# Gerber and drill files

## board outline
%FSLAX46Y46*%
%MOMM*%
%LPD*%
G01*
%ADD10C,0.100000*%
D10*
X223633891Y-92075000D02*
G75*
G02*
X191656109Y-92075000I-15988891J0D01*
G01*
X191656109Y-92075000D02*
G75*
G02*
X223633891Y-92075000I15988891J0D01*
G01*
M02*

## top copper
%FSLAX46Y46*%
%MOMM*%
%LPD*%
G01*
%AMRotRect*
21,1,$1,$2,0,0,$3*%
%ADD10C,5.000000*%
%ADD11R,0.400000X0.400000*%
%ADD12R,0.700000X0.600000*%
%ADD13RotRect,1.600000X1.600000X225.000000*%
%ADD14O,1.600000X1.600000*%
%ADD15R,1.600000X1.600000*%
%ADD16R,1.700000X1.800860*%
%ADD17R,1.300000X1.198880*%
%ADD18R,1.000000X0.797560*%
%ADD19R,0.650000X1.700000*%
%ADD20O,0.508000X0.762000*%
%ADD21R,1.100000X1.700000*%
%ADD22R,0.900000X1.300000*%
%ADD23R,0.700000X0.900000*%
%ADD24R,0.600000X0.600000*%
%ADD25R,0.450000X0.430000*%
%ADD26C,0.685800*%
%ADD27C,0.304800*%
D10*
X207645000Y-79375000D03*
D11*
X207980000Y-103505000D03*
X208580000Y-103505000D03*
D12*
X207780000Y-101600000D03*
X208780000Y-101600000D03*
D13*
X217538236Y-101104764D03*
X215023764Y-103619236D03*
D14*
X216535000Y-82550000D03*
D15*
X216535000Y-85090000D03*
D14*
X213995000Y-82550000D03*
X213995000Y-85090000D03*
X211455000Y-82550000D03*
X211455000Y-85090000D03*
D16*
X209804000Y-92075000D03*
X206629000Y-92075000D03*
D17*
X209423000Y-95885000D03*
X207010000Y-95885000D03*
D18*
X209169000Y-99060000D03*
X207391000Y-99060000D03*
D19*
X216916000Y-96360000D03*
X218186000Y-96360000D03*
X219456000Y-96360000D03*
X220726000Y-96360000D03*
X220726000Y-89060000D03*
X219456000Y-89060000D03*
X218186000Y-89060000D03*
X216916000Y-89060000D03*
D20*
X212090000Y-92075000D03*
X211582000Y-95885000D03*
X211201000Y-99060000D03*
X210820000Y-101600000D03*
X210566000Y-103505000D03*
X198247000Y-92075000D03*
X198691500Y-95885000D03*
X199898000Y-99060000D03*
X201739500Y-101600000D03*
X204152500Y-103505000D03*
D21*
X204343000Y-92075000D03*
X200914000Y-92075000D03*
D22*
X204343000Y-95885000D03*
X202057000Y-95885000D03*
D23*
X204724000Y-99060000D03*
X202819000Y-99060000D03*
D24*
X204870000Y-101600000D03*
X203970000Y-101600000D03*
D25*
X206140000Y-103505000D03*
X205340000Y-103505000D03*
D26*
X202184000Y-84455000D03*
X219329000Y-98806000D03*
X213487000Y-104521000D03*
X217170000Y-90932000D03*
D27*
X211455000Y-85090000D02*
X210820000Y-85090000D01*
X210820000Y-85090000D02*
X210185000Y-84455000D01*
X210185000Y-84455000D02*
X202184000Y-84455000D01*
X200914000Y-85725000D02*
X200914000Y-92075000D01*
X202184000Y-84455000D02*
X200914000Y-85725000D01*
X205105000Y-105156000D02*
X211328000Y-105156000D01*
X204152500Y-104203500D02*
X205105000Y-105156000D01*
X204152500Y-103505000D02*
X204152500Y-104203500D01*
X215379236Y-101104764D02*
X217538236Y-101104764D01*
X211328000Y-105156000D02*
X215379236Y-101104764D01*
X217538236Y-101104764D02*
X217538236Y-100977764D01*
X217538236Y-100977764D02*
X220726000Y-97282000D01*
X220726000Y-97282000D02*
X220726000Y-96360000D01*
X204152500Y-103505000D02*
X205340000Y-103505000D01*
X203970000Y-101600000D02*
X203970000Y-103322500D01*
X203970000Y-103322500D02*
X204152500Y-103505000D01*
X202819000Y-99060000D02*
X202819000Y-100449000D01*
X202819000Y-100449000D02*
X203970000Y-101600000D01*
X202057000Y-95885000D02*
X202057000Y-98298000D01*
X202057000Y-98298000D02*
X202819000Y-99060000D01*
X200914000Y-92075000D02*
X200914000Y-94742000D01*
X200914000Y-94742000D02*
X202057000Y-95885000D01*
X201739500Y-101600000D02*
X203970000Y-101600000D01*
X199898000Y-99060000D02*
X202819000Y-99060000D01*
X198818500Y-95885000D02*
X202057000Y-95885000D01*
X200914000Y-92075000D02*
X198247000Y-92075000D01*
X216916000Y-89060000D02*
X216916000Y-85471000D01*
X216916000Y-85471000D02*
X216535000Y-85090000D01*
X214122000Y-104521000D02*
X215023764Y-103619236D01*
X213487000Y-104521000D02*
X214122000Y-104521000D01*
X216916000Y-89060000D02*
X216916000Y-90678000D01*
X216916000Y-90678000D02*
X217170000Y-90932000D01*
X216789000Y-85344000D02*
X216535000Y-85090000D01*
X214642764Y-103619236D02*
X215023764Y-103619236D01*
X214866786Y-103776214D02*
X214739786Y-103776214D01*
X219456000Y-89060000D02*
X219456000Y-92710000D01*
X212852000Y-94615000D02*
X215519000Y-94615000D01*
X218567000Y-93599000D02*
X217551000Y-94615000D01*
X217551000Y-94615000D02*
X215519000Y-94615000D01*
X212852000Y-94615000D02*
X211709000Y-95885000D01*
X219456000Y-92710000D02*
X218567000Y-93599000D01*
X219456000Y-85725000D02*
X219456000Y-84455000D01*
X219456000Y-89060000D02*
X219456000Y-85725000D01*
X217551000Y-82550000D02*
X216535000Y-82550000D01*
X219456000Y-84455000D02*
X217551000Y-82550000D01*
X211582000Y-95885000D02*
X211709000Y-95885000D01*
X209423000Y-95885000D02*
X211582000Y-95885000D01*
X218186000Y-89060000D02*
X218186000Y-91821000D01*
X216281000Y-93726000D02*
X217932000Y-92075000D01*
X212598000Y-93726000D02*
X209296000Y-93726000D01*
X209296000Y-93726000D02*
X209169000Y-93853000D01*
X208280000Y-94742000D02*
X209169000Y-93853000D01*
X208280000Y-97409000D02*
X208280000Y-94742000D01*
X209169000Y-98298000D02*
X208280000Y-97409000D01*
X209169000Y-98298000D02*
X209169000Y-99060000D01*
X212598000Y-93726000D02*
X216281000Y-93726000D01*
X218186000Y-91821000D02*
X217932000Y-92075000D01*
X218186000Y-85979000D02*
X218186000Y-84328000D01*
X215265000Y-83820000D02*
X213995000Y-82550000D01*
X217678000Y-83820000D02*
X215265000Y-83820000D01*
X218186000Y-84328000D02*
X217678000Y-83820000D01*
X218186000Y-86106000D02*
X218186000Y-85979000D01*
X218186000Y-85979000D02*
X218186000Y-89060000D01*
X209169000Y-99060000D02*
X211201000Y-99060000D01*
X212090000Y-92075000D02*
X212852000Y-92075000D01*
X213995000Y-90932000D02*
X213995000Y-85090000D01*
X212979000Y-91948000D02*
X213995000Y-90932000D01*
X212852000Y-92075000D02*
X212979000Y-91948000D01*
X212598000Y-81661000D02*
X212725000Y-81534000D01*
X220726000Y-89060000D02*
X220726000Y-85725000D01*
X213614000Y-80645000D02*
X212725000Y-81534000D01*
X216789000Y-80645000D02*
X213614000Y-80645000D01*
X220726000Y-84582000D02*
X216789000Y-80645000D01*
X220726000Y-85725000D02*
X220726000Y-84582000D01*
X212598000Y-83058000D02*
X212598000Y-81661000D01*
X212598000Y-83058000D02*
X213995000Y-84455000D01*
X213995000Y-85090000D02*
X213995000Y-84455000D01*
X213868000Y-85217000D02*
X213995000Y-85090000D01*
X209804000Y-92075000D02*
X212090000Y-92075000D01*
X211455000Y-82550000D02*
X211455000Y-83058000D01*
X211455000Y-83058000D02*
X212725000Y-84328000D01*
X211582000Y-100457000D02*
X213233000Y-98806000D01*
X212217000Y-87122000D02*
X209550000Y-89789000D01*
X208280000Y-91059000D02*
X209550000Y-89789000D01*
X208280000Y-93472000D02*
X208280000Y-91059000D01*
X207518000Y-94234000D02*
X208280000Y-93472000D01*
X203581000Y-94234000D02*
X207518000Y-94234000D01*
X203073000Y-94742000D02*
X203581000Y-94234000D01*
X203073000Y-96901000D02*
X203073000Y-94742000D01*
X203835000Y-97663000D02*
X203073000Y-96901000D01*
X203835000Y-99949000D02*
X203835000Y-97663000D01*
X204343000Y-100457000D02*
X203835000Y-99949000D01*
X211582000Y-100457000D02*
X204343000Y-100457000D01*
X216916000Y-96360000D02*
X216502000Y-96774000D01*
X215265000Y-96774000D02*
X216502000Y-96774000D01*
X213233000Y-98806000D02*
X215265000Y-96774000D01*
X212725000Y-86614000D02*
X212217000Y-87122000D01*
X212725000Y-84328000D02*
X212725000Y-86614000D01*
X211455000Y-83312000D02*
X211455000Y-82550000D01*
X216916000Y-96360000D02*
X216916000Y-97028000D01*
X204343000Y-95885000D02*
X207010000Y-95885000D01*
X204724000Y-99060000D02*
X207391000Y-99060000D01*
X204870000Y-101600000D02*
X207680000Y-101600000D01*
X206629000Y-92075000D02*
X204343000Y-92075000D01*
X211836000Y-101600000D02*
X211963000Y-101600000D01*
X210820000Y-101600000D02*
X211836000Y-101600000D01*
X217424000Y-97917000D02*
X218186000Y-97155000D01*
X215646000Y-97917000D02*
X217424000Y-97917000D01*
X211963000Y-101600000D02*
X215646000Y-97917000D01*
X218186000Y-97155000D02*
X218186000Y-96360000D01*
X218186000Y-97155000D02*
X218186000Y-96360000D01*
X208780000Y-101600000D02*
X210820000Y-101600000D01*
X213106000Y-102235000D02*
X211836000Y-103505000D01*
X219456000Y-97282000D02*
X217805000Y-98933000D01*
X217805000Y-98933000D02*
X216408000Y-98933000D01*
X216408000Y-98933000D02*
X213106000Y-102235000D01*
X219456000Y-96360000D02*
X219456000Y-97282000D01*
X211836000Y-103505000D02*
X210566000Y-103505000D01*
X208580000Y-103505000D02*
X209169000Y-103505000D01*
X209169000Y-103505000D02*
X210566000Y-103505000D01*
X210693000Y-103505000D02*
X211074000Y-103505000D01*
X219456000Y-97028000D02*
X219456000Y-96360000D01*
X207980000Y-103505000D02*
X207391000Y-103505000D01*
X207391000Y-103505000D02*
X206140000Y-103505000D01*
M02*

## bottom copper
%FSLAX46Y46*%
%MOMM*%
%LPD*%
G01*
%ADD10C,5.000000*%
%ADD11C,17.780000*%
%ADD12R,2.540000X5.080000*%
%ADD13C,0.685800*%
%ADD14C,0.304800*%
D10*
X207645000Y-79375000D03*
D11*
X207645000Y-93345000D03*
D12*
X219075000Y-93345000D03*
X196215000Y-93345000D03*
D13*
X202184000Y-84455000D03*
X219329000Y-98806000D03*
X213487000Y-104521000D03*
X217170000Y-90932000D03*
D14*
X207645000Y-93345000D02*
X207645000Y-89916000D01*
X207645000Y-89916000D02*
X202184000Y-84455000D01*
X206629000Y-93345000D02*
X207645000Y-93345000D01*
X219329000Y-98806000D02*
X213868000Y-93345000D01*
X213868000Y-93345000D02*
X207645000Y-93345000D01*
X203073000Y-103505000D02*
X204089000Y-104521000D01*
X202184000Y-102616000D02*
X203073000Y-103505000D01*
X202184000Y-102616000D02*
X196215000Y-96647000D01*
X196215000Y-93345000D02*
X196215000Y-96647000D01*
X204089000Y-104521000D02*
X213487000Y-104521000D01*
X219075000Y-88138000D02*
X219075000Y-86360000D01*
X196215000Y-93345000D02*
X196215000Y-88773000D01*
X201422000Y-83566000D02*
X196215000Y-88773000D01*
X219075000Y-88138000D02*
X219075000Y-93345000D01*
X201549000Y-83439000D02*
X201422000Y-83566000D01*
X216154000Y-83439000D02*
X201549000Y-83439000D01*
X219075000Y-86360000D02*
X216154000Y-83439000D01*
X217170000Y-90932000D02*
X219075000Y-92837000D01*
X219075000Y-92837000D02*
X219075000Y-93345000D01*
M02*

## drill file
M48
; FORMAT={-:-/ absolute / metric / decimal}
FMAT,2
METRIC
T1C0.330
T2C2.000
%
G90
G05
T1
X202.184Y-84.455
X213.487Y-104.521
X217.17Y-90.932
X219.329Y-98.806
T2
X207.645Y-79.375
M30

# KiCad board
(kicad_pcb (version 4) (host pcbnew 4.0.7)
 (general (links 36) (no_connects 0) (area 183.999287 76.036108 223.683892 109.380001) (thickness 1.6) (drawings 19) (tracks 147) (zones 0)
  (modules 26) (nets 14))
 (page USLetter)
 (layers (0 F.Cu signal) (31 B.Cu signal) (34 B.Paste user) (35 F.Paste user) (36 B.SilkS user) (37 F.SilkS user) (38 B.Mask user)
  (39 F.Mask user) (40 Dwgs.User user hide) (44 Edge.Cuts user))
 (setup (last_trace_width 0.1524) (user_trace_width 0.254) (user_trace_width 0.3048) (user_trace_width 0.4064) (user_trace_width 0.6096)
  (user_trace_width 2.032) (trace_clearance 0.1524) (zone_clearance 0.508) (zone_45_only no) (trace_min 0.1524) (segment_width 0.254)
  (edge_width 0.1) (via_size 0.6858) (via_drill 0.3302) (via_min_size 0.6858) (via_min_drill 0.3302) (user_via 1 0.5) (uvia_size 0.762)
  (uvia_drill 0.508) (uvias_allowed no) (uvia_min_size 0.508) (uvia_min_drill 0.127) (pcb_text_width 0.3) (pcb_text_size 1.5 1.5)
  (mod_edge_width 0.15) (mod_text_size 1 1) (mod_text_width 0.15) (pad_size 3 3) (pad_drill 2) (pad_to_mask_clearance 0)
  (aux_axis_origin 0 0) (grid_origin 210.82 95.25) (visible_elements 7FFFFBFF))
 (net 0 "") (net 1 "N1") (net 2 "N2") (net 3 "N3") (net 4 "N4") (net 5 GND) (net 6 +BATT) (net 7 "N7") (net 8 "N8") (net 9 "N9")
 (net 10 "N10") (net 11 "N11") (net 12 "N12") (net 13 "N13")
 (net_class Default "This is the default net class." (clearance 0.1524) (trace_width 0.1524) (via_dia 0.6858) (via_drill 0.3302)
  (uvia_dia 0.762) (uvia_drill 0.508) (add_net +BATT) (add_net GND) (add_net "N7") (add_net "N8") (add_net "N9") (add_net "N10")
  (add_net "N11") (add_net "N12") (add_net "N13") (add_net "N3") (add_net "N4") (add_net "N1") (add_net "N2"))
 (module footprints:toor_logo (layer F.Cu) (at 205.232 88.392)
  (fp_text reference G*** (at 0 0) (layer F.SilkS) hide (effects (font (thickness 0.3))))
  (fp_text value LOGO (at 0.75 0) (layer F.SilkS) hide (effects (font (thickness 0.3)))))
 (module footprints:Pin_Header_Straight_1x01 (layer F.Cu) (at 207.645 79.375)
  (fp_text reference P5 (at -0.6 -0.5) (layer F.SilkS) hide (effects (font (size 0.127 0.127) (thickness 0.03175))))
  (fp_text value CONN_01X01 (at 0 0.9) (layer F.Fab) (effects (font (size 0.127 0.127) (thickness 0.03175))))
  (pad 1 thru_hole circle (at 0 0) (size 5 5) (drill 2) (layers *.Cu *.Mask)))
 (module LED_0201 (layer F.Cu) (at 208.28 103.505)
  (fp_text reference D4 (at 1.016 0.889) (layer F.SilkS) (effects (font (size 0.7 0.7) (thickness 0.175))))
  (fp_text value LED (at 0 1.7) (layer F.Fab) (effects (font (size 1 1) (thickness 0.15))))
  (pad 1 smd rect (at -0.3 0) (size 0.4 0.4) (layers F.Cu F.Paste F.Mask) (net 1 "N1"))
  (pad 2 smd rect (at 0.3 0) (size 0.4 0.4) (layers F.Cu F.Paste F.Mask) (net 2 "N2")))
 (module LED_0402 (layer F.Cu) (at 208.28 101.6)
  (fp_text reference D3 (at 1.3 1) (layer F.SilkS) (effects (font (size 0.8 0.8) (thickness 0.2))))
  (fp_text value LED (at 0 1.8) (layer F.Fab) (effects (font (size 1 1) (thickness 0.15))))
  (pad 1 smd rect (at -0.5 0) (size 0.7 0.6) (layers F.Cu F.Paste F.Mask) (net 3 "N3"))
  (pad 2 smd rect (at 0.5 0) (size 0.7 0.6) (layers F.Cu F.Paste F.Mask) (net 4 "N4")))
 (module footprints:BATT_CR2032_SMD (layer B.Cu) (at 207.645 93.345 180)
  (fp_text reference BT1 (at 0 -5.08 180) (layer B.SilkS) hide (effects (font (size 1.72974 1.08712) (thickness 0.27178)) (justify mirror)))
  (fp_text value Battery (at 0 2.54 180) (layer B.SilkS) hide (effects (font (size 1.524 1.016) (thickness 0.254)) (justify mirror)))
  (pad 2 smd circle (at 0 0 180) (size 17.78 17.78) (layers B.Cu B.Paste B.Mask) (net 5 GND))
  (pad 1 smd rect (at -11.43 0 180) (size 2.54 5.08) (layers B.Cu B.Paste B.Mask) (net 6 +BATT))
  (pad 1 smd rect (at 11.43 0 180) (size 2.54 5.08) (layers B.Cu B.Paste B.Mask) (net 6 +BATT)))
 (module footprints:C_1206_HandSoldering (layer F.Cu) (at 216.281 102.362 225)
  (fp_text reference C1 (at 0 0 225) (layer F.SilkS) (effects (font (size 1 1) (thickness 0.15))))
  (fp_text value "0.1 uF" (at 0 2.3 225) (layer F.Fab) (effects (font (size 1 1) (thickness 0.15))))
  (pad 1 smd rect (at -1.778 0 225) (size 1.6 1.6) (layers F.Cu F.Paste F.Mask) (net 5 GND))
  (pad 2 smd rect (at 1.778 0 225) (size 1.6 1.6) (layers F.Cu F.Paste F.Mask) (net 6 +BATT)))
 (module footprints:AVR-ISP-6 (layer F.Cu) (at 216.535 82.55 270)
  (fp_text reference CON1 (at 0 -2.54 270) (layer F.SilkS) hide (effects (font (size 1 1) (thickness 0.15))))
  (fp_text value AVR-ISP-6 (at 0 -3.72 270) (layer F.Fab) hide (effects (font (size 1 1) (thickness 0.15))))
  (pad 1 smd oval (at 0 0 270) (size 1.6 1.6) (layers F.Cu F.Paste F.Mask) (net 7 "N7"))
  (pad 2 smd rect (at 2.54 0 270) (size 1.6 1.6) (layers F.Cu F.Paste F.Mask) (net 6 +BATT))
  (pad 3 smd oval (at 0 2.54 270) (size 1.6 1.6) (layers F.Cu F.Paste F.Mask) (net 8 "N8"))
  (pad 4 smd oval (at 2.54 2.54 270) (size 1.6 1.6) (layers F.Cu F.Paste F.Mask) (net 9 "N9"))
  (pad 5 smd oval (at 0 5.08 270) (size 1.6 1.6) (layers F.Cu F.Paste F.Mask) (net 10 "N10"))
  (pad 6 smd oval (at 2.54 5.08 270) (size 1.6 1.6) (layers F.Cu F.Paste F.Mask) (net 5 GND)))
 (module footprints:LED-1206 (layer F.Cu) (at 208.28 92.075)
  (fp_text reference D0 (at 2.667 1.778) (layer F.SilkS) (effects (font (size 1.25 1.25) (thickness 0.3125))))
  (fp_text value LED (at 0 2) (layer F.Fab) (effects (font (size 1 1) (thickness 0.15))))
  (pad 2 smd rect (at 1.524 0 180) (size 1.7 1.80086) (layers F.Cu F.Paste F.Mask) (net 9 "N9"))
  (pad 1 smd rect (at -1.651 0 180) (size 1.7 1.80086) (layers F.Cu F.Paste F.Mask) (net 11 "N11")))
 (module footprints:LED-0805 (layer F.Cu) (at 208.28 95.885)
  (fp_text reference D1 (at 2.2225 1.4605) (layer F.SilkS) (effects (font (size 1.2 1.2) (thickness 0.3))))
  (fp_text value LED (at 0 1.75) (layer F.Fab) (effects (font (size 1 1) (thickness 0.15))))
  (pad 2 smd rect (at 1.143 0 180) (size 1.3 1.19888) (layers F.Cu F.Paste F.Mask) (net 7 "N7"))
  (pad 1 smd rect (at -1.27 0 180) (size 1.3 1.19888) (layers F.Cu F.Paste F.Mask) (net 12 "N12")))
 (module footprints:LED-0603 (layer F.Cu) (at 208.28 99.06)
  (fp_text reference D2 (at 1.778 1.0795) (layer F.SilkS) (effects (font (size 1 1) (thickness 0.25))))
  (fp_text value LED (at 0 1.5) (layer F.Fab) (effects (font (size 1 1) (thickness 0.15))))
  (pad 2 smd rect (at 0.889 0 180) (size 1 0.79756) (layers F.Cu F.Paste F.Mask) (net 8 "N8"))
  (pad 1 smd rect (at -0.889 0 180) (size 1 0.79756) (layers F.Cu F.Paste F.Mask) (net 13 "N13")))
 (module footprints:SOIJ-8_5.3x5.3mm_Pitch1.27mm (layer F.Cu) (at 218.821 92.71 90)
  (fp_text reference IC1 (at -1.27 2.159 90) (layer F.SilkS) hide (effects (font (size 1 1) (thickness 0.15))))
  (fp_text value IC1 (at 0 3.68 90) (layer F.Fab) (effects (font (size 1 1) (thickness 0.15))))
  (pad 1 smd rect (at -3.65 -1.905 90) (size 1.7 0.65) (layers F.Cu F.Paste F.Mask) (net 10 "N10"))
  (pad 2 smd rect (at -3.65 -0.635 90) (size 1.7 0.65) (layers F.Cu F.Paste F.Mask) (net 4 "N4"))
  (pad 3 smd rect (at -3.65 0.635 90) (size 1.7 0.65) (layers F.Cu F.Paste F.Mask) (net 2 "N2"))
  (pad 4 smd rect (at -3.65 1.905 90) (size 1.7 0.65) (layers F.Cu F.Paste F.Mask) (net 5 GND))
  (pad 5 smd rect (at 3.65 1.905 90) (size 1.7 0.65) (layers F.Cu F.Paste F.Mask) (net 9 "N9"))
  (pad 6 smd rect (at 3.65 0.635 90) (size 1.7 0.65) (layers F.Cu F.Paste F.Mask) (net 7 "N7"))
  (pad 7 smd rect (at 3.65 -0.635 90) (size 1.7 0.65) (layers F.Cu F.Paste F.Mask) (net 8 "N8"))
  (pad 8 smd rect (at 3.65 -1.905 90) (size 1.7 0.65) (layers F.Cu F.Paste F.Mask) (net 6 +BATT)))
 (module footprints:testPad (layer F.Cu) (at 212.09 92.075)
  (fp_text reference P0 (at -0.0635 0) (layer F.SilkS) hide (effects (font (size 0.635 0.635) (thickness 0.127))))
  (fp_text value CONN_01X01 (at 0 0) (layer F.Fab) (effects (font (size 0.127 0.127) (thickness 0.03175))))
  (pad 1 smd oval (at 0 0) (size 0.508 0.762) (layers F.Cu F.Paste F.Mask) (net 9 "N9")))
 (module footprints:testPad (layer F.Cu) (at 211.582 95.885)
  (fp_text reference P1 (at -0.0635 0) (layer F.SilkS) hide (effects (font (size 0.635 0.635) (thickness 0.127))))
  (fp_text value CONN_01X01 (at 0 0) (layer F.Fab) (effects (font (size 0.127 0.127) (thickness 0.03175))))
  (pad 1 smd oval (at 0 0) (size 0.508 0.762) (layers F.Cu F.Paste F.Mask) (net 7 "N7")))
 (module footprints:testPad (layer F.Cu) (at 211.201 99.06)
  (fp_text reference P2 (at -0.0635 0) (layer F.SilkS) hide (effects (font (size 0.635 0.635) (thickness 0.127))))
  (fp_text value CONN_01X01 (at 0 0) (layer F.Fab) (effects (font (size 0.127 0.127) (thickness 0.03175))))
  (pad 1 smd oval (at 0 0) (size 0.508 0.762) (layers F.Cu F.Paste F.Mask) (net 8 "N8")))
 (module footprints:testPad (layer F.Cu) (at 210.82 101.6)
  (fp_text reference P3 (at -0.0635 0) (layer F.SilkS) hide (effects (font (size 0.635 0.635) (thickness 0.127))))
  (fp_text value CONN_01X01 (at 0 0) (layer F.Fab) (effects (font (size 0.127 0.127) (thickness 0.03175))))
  (pad 1 smd oval (at 0 0) (size 0.508 0.762) (layers F.Cu F.Paste F.Mask) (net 4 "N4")))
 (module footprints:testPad (layer F.Cu) (at 210.566 103.505)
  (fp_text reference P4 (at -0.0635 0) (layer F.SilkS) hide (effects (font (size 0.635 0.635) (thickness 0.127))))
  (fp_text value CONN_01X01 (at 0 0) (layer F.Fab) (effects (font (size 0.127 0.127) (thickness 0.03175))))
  (pad 1 smd oval (at 0 0) (size 0.508 0.762) (layers F.Cu F.Paste F.Mask) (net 2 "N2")))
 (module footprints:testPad (layer F.Cu) (at 198.247 92.075)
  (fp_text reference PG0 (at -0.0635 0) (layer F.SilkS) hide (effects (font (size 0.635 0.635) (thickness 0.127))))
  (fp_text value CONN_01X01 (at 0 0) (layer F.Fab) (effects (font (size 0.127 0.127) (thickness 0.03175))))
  (pad 1 smd oval (at 0 0) (size 0.508 0.762) (layers F.Cu F.Paste F.Mask) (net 5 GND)))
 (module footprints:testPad (layer F.Cu) (at 198.6915 95.885)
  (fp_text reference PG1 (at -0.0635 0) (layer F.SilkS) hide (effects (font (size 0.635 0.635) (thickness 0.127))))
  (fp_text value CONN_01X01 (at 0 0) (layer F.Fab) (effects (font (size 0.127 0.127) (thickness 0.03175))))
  (pad 1 smd oval (at 0 0) (size 0.508 0.762) (layers F.Cu F.Paste F.Mask) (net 5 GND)))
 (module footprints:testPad (layer F.Cu) (at 199.898 99.06)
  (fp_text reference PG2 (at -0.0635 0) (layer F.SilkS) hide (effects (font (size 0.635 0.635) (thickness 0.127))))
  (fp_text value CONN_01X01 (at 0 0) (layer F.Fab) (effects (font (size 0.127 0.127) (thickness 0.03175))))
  (pad 1 smd oval (at 0 0) (size 0.508 0.762) (layers F.Cu F.Paste F.Mask) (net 5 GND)))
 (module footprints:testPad (layer F.Cu) (at 201.7395 101.6)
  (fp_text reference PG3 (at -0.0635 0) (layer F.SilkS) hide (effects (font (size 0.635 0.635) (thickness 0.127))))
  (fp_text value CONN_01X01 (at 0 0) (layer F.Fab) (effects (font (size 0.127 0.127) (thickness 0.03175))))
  (pad 1 smd oval (at 0 0) (size 0.508 0.762) (layers F.Cu F.Paste F.Mask) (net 5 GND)))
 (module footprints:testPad (layer F.Cu) (at 204.1525 103.505)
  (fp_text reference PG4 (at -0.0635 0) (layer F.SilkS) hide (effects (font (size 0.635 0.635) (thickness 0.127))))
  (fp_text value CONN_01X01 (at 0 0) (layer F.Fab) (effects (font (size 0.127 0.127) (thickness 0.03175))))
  (pad 1 smd oval (at 0 0) (size 0.508 0.762) (layers F.Cu F.Paste F.Mask) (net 5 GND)))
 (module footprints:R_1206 (layer F.Cu) (at 202.565 92.075 180)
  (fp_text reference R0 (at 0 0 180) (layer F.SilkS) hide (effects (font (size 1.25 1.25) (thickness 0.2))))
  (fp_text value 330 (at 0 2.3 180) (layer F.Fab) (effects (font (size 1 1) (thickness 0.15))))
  (pad 1 smd rect (at -1.778 0 180) (size 1.1 1.7) (layers F.Cu F.Paste F.Mask) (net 11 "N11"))
  (pad 2 smd rect (at 1.651 0 180) (size 1.1 1.7) (layers F.Cu F.Paste F.Mask) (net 5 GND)))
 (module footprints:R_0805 (layer F.Cu) (at 203.2 95.885 180)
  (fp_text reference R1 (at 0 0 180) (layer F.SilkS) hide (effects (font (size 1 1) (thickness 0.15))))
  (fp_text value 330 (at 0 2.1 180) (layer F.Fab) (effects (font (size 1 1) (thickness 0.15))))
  (pad 1 smd rect (at -1.143 0 180) (size 0.9 1.3) (layers F.Cu F.Paste F.Mask) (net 12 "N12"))
  (pad 2 smd rect (at 1.143 0 180) (size 0.9 1.3) (layers F.Cu F.Paste F.Mask) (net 5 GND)))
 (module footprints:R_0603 (layer F.Cu) (at 203.835 99.06 180)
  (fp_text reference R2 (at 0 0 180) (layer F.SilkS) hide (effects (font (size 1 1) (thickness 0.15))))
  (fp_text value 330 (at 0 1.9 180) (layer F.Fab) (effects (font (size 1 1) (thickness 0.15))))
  (pad 1 smd rect (at -0.889 0 180) (size 0.7 0.9) (layers F.Cu F.Paste F.Mask) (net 13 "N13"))
  (pad 2 smd rect (at 1.016 0 180) (size 0.7 0.9) (layers F.Cu F.Paste F.Mask) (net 5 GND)))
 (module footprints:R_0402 (layer F.Cu) (at 204.47 101.6 180)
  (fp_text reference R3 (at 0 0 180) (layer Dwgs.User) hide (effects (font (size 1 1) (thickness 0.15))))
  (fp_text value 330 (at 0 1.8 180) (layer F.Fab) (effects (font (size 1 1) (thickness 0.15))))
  (pad 1 smd rect (at -0.4 0 180) (size 0.6 0.6) (layers F.Cu F.Paste F.Mask) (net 3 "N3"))
  (pad 2 smd rect (at 0.5 0 180) (size 0.6 0.6) (layers F.Cu F.Paste F.Mask) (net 5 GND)))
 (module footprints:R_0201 (layer F.Cu) (at 205.74 103.505 180)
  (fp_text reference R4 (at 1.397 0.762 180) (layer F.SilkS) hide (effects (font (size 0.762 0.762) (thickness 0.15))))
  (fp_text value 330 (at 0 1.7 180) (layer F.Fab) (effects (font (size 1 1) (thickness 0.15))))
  (pad 1 smd rect (at -0.4 0 180) (size 0.45 0.43) (layers F.Cu F.Paste F.Mask) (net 1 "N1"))
  (pad 2 smd rect (at 0.4 0 180) (size 0.45 0.43) (layers F.Cu F.Paste F.Mask) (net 5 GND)))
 (gr_circle (center 207.645 92.075) (end 191.77 90.17) (layer Edge.Cuts) (width 0.1))
 (segment (start 211.455 85.09) (end 210.82 85.09) (width 0.3048) (layer F.Cu) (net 5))
 (segment (start 210.82 85.09) (end 210.185 84.455) (width 0.3048) (layer F.Cu) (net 5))
 (segment (start 210.185 84.455) (end 202.184 84.455) (width 0.3048) (layer F.Cu) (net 5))
 (segment (start 207.645 93.345) (end 207.645 89.916) (width 0.3048) (layer B.Cu) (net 5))
 (segment (start 207.645 89.916) (end 202.184 84.455) (width 0.3048) (layer B.Cu) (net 5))
 (segment (start 200.914 85.725) (end 200.914 92.075) (width 0.3048) (layer F.Cu) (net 5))
 (segment (start 202.184 84.455) (end 200.914 85.725) (width 0.3048) (layer F.Cu) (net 5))
 (via (at 202.184 84.455) (size 0.6858) (drill 0.3302) (layers F.Cu B.Cu) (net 5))
 (segment (start 205.105 105.156) (end 211.328 105.156) (width 0.3048) (layer F.Cu) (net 5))
 (segment (start 204.1525 104.2035) (end 205.105 105.156) (width 0.3048) (layer F.Cu) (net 5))
 (segment (start 204.1525 103.505) (end 204.1525 104.2035) (width 0.3048) (layer F.Cu) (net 5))
 (segment (start 215.379236 101.104764) (end 217.538236 101.104764) (width 0.3048) (layer F.Cu) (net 5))
 (segment (start 211.328 105.156) (end 215.379236 101.104764) (width 0.3048) (layer F.Cu) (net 5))
 (segment (start 217.538236 101.104764) (end 217.538236 100.977764) (width 0.3048) (layer F.Cu) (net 5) (status 30))
 (segment (start 217.538236 100.977764) (end 220.726 97.282) (width 0.3048) (layer F.Cu) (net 5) (status 10))
 (segment (start 220.726 97.282) (end 220.726 96.36) (width 0.3048) (layer F.Cu) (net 5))
 (segment (start 204.1525 103.505) (end 205.34 103.505) (width 0.3048) (layer F.Cu) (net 5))
 (segment (start 203.97 101.6) (end 203.97 103.3225) (width 0.3048) (layer F.Cu) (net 5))
 (segment (start 203.97 103.3225) (end 204.1525 103.505) (width 0.3048) (layer F.Cu) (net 5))
 (segment (start 206.629 93.345) (end 207.645 93.345) (width 0.3048) (layer B.Cu) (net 5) (status 30))
 (segment (start 219.329 98.806) (end 213.868 93.345) (width 0.3048) (layer B.Cu) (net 5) (status 20))
 (via (at 219.329 98.806) (size 0.6858) (drill 0.3302) (layers F.Cu B.Cu) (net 5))
 (segment (start 213.868 93.345) (end 207.645 93.345) (width 0.3048) (layer B.Cu) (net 5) (status 30))
 (segment (start 202.819 99.06) (end 202.819 100.449) (width 0.3048) (layer F.Cu) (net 5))
 (segment (start 202.819 100.449) (end 203.97 101.6) (width 0.3048) (layer F.Cu) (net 5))
 (segment (start 202.057 95.885) (end 202.057 98.298) (width 0.3048) (layer F.Cu) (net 5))
 (segment (start 202.057 98.298) (end 202.819 99.06) (width 0.3048) (layer F.Cu) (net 5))
 (segment (start 200.914 92.075) (end 200.914 94.742) (width 0.3048) (layer F.Cu) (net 5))
 (segment (start 200.914 94.742) (end 202.057 95.885) (width 0.3048) (layer F.Cu) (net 5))
 (segment (start 201.7395 101.6) (end 203.97 101.6) (width 0.3048) (layer F.Cu) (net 5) (status 10))
 (segment (start 199.898 99.06) (end 202.819 99.06) (width 0.3048) (layer F.Cu) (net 5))
 (segment (start 198.8185 95.885) (end 202.057 95.885) (width 0.3048) (layer F.Cu) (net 5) (status 10))
 (segment (start 200.914 92.075) (end 198.247 92.075) (width 0.3048) (layer F.Cu) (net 5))
 (segment (start 216.916 89.06) (end 216.916 85.471) (width 0.3048) (layer F.Cu) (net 6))
 (segment (start 216.916 85.471) (end 216.535 85.09) (width 0.3048) (layer F.Cu) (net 6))
 (segment (start 203.073 103.505) (end 204.089 104.521) (width 0.3048) (layer B.Cu) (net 6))
 (segment (start 202.184 102.616) (end 203.073 103.505) (width 0.3048) (layer B.Cu) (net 6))
 (segment (start 202.184 102.616) (end 196.215 96.647) (width 0.3048) (layer B.Cu) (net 6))
 (segment (start 196.215 93.345) (end 196.215 96.647) (width 0.3048) (layer B.Cu) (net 6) (status 10))
 (segment (start 214.122 104.521) (end 215.023764 103.619236) (width 0.3048) (layer F.Cu) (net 6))
 (segment (start 213.487 104.521) (end 214.122 104.521) (width 0.3048) (layer F.Cu) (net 6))
 (via (at 213.487 104.521) (size 0.6858) (drill 0.3302) (layers F.Cu B.Cu) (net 6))
 (segment (start 204.089 104.521) (end 213.487 104.521) (width 0.3048) (layer B.Cu) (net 6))
 (segment (start 219.075 88.138) (end 219.075 86.36) (width 0.3048) (layer B.Cu) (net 6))
 (segment (start 196.215 93.345) (end 196.215 88.773) (width 0.3048) (layer B.Cu) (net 6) (status 20))
 (segment (start 201.422 83.566) (end 196.215 88.773) (width 0.3048) (layer B.Cu) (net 6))
 (segment (start 219.075 88.138) (end 219.075 93.345) (width 0.3048) (layer B.Cu) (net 6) (status 10))
 (segment (start 201.549 83.439) (end 201.422 83.566) (width 0.3048) (layer B.Cu) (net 6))
 (segment (start 216.154 83.439) (end 201.549 83.439) (width 0.3048) (layer B.Cu) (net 6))
 (segment (start 219.075 86.36) (end 216.154 83.439) (width 0.3048) (layer B.Cu) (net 6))
 (segment (start 216.916 89.06) (end 216.916 90.678) (width 0.3048) (layer F.Cu) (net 6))
 (segment (start 217.17 90.932) (end 219.075 92.837) (width 0.3048) (layer B.Cu) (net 6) (status 20))
 (via (at 217.17 90.932) (size 0.6858) (drill 0.3302) (layers F.Cu B.Cu) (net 6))
 (segment (start 216.916 90.678) (end 217.17 90.932) (width 0.3048) (layer F.Cu) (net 6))
 (segment (start 216.789 85.344) (end 216.535 85.09) (width 0.3048) (layer F.Cu) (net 6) (status 30))
 (segment (start 214.642764 103.619236) (end 215.023764 103.619236) (width 0.3048) (layer F.Cu) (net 6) (status 30))
 (segment (start 219.075 92.837) (end 219.075 93.345) (width 0.3048) (layer B.Cu) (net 6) (status 30))
 (segment (start 214.866786 103.776214) (end 214.739786 103.776214) (width 0.3048) (layer F.Cu) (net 6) (status 30))
 (segment (start 219.456 89.06) (end 219.456 92.71) (width 0.3048) (layer F.Cu) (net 7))
 (segment (start 212.852 94.615) (end 215.519 94.615) (width 0.3048) (layer F.Cu) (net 7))
 (segment (start 218.567 93.599) (end 217.551 94.615) (width 0.3048) (layer F.Cu) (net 7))
 (segment (start 217.551 94.615) (end 215.519 94.615) (width 0.3048) (layer F.Cu) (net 7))
 (segment (start 212.852 94.615) (end 211.709 95.885) (width 0.3048) (layer F.Cu) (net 7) (status 20))
 (segment (start 219.456 92.71) (end 218.567 93.599) (width 0.3048) (layer F.Cu) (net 7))
 (segment (start 219.456 85.725) (end 219.456 84.455) (width 0.3048) (layer F.Cu) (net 7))
 (segment (start 219.456 89.06) (end 219.456 85.725) (width 0.3048) (layer F.Cu) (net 7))
 (segment (start 217.551 82.55) (end 216.535 82.55) (width 0.3048) (layer F.Cu) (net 7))
 (segment (start 219.456 84.455) (end 217.551 82.55) (width 0.3048) (layer F.Cu) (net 7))
 (segment (start 211.582 95.885) (end 211.709 95.885) (width 0.3048) (layer F.Cu) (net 7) (status 30))
 (segment (start 209.423 95.885) (end 211.582 95.885) (width 0.3048) (layer F.Cu) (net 7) (status 20))
 (segment (start 218.186 89.06) (end 218.186 91.821) (width 0.3048) (layer F.Cu) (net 8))
 (segment (start 216.281 93.726) (end 217.932 92.075) (width 0.3048) (layer F.Cu) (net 8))
 (segment (start 212.598 93.726) (end 209.296 93.726) (width 0.3048) (layer F.Cu) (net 8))
 (segment (start 209.296 93.726) (end 209.169 93.853) (width 0.3048) (layer F.Cu) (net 8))
 (segment (start 208.28 94.742) (end 209.169 93.853) (width 0.3048) (layer F.Cu) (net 8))
 (segment (start 208.28 97.409) (end 208.28 94.742) (width 0.3048) (layer F.Cu) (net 8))
 (segment (start 209.169 98.298) (end 208.28 97.409) (width 0.3048) (layer F.Cu) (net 8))
 (segment (start 209.169 98.298) (end 209.169 99.06) (width 0.3048) (layer F.Cu) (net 8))
 (segment (start 212.598 93.726) (end 216.281 93.726) (width 0.3048) (layer F.Cu) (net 8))
 (segment (start 218.186 91.821) (end 217.932 92.075) (width 0.3048) (layer F.Cu) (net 8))
 (segment (start 218.186 85.979) (end 218.186 84.328) (width 0.3048) (layer F.Cu) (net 8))
 (segment (start 215.265 83.82) (end 213.995 82.55) (width 0.3048) (layer F.Cu) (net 8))
 (segment (start 217.678 83.82) (end 215.265 83.82) (width 0.3048) (layer F.Cu) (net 8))
 (segment (start 218.186 84.328) (end 217.678 83.82) (width 0.3048) (layer F.Cu) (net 8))
 (segment (start 218.186 86.106) (end 218.186 85.979) (width 0.3048) (layer F.Cu) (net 8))
 (segment (start 218.186 85.979) (end 218.186 89.06) (width 0.3048) (layer F.Cu) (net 8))
 (segment (start 209.169 99.06) (end 211.201 99.06) (width 0.3048) (layer F.Cu) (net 8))
 (segment (start 212.09 92.075) (end 212.852 92.075) (width 0.3048) (layer F.Cu) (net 9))
 (segment (start 213.995 90.932) (end 213.995 85.09) (width 0.3048) (layer F.Cu) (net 9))
 (segment (start 212.979 91.948) (end 213.995 90.932) (width 0.3048) (layer F.Cu) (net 9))
 (segment (start 212.852 92.075) (end 212.979 91.948) (width 0.3048) (layer F.Cu) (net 9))
 (segment (start 212.598 81.661) (end 212.725 81.534) (width 0.3048) (layer F.Cu) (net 9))
 (segment (start 220.726 89.06) (end 220.726 85.725) (width 0.3048) (layer F.Cu) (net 9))
 (segment (start 213.614 80.645) (end 212.725 81.534) (width 0.3048) (layer F.Cu) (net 9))
 (segment (start 216.789 80.645) (end 213.614 80.645) (width 0.3048) (layer F.Cu) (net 9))
 (segment (start 220.726 84.582) (end 216.789 80.645) (width 0.3048) (layer F.Cu) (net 9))
 (segment (start 220.726 85.725) (end 220.726 84.582) (width 0.3048) (layer F.Cu) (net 9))
 (segment (start 212.598 83.058) (end 212.598 81.661) (width 0.3048) (layer F.Cu) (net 9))
 (segment (start 212.598 83.058) (end 213.995 84.455) (width 0.3048) (layer F.Cu) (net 9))
 (segment (start 213.995 85.09) (end 213.995 84.455) (width 0.3048) (layer F.Cu) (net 9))
 (segment (start 213.868 85.217) (end 213.995 85.09) (width 0.3048) (layer F.Cu) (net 9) (status 30))
 (segment (start 209.804 92.075) (end 212.09 92.075) (width 0.3048) (layer F.Cu) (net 9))
 (segment (start 211.455 82.55) (end 211.455 83.058) (width 0.3048) (layer F.Cu) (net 10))
 (segment (start 211.455 83.058) (end 212.725 84.328) (width 0.3048) (layer F.Cu) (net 10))
 (segment (start 211.582 100.457) (end 213.233 98.806) (width 0.3048) (layer F.Cu) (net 10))
 (segment (start 212.217 87.122) (end 209.55 89.789) (width 0.3048) (layer F.Cu) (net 10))
 (segment (start 208.28 91.059) (end 209.55 89.789) (width 0.3048) (layer F.Cu) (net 10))
 (segment (start 208.28 93.472) (end 208.28 91.059) (width 0.3048) (layer F.Cu) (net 10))
 (segment (start 207.518 94.234) (end 208.28 93.472) (width 0.3048) (layer F.Cu) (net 10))
 (segment (start 203.581 94.234) (end 207.518 94.234) (width 0.3048) (layer F.Cu) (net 10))
 (segment (start 203.073 94.742) (end 203.581 94.234) (width 0.3048) (layer F.Cu) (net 10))
 (segment (start 203.073 96.901) (end 203.073 94.742) (width 0.3048) (layer F.Cu) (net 10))
 (segment (start 203.835 97.663) (end 203.073 96.901) (width 0.3048) (layer F.Cu) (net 10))
 (segment (start 203.835 99.949) (end 203.835 97.663) (width 0.3048) (layer F.Cu) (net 10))
 (segment (start 204.343 100.457) (end 203.835 99.949) (width 0.3048) (layer F.Cu) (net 10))
 (segment (start 211.582 100.457) (end 204.343 100.457) (width 0.3048) (layer F.Cu) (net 10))
 (segment (start 216.916 96.36) (end 216.502 96.774) (width 0.3048) (layer F.Cu) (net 10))
 (segment (start 215.265 96.774) (end 216.502 96.774) (width 0.3048) (layer F.Cu) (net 10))
 (segment (start 213.233 98.806) (end 215.265 96.774) (width 0.3048) (layer F.Cu) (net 10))
 (segment (start 212.725 86.614) (end 212.217 87.122) (width 0.3048) (layer F.Cu) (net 10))
 (segment (start 212.725 84.328) (end 212.725 86.614) (width 0.3048) (layer F.Cu) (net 10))
 (segment (start 211.455 83.312) (end 211.455 82.55) (width 0.3048) (layer F.Cu) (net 10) (status 30))
 (segment (start 216.916 96.36) (end 216.916 97.028) (width 0.3048) (layer F.Cu) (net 10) (status 30))
 (segment (start 204.343 95.885) (end 207.01 95.885) (width 0.3048) (layer F.Cu) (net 12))
 (segment (start 204.724 99.06) (end 207.391 99.06) (width 0.3048) (layer F.Cu) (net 13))
 (segment (start 204.87 101.6) (end 207.68 101.6) (width 0.3048) (layer F.Cu) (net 3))
 (segment (start 206.629 92.075) (end 204.343 92.075) (width 0.3048) (layer F.Cu) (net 11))
 (segment (start 211.836 101.6) (end 211.963 101.6) (width 0.3048) (layer F.Cu) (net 4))
 (segment (start 210.82 101.6) (end 211.836 101.6) (width 0.3048) (layer F.Cu) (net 4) (status 10))
 (segment (start 217.424 97.917) (end 218.186 97.155) (width 0.3048) (layer F.Cu) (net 4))
 (segment (start 215.646 97.917) (end 217.424 97.917) (width 0.3048) (layer F.Cu) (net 4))
 (segment (start 211.963 101.6) (end 215.646 97.917) (width 0.3048) (layer F.Cu) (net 4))
 (segment (start 218.186 97.155) (end 218.186 96.36) (width 0.3048) (layer F.Cu) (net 4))
 (segment (start 218.186 97.155) (end 218.186 96.36) (width 0.3048) (layer F.Cu) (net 4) (status 30))
 (segment (start 208.78 101.6) (end 210.82 101.6) (width 0.3048) (layer F.Cu) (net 4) (status 20))
 (segment (start 213.106 102.235) (end 211.836 103.505) (width 0.3048) (layer F.Cu) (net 2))
 (segment (start 219.456 97.282) (end 217.805 98.933) (width 0.3048) (layer F.Cu) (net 2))
 (segment (start 217.805 98.933) (end 216.408 98.933) (width 0.3048) (layer F.Cu) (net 2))
 (segment (start 216.408 98.933) (end 213.106 102.235) (width 0.3048) (layer F.Cu) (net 2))
 (segment (start 219.456 96.36) (end 219.456 97.282) (width 0.3048) (layer F.Cu) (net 2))
 (segment (start 211.836 103.505) (end 210.566 103.505) (width 0.3048) (layer F.Cu) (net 2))
 (segment (start 208.58 103.505) (end 209.169 103.505) (width 0.3048) (layer F.Cu) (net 2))
 (segment (start 209.169 103.505) (end 210.566 103.505) (width 0.3048) (layer F.Cu) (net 2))
 (segment (start 210.693 103.505) (end 211.074 103.505) (width 0.3048) (layer F.Cu) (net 2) (status 10))
 (segment (start 219.456 97.028) (end 219.456 96.36) (width 0.3048) (layer F.Cu) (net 2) (status 30))
 (segment (start 207.98 103.505) (end 207.391 103.505) (width 0.3048) (layer F.Cu) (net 1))
 (segment (start 207.391 103.505) (end 206.14 103.505) (width 0.3048) (layer F.Cu) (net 1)))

